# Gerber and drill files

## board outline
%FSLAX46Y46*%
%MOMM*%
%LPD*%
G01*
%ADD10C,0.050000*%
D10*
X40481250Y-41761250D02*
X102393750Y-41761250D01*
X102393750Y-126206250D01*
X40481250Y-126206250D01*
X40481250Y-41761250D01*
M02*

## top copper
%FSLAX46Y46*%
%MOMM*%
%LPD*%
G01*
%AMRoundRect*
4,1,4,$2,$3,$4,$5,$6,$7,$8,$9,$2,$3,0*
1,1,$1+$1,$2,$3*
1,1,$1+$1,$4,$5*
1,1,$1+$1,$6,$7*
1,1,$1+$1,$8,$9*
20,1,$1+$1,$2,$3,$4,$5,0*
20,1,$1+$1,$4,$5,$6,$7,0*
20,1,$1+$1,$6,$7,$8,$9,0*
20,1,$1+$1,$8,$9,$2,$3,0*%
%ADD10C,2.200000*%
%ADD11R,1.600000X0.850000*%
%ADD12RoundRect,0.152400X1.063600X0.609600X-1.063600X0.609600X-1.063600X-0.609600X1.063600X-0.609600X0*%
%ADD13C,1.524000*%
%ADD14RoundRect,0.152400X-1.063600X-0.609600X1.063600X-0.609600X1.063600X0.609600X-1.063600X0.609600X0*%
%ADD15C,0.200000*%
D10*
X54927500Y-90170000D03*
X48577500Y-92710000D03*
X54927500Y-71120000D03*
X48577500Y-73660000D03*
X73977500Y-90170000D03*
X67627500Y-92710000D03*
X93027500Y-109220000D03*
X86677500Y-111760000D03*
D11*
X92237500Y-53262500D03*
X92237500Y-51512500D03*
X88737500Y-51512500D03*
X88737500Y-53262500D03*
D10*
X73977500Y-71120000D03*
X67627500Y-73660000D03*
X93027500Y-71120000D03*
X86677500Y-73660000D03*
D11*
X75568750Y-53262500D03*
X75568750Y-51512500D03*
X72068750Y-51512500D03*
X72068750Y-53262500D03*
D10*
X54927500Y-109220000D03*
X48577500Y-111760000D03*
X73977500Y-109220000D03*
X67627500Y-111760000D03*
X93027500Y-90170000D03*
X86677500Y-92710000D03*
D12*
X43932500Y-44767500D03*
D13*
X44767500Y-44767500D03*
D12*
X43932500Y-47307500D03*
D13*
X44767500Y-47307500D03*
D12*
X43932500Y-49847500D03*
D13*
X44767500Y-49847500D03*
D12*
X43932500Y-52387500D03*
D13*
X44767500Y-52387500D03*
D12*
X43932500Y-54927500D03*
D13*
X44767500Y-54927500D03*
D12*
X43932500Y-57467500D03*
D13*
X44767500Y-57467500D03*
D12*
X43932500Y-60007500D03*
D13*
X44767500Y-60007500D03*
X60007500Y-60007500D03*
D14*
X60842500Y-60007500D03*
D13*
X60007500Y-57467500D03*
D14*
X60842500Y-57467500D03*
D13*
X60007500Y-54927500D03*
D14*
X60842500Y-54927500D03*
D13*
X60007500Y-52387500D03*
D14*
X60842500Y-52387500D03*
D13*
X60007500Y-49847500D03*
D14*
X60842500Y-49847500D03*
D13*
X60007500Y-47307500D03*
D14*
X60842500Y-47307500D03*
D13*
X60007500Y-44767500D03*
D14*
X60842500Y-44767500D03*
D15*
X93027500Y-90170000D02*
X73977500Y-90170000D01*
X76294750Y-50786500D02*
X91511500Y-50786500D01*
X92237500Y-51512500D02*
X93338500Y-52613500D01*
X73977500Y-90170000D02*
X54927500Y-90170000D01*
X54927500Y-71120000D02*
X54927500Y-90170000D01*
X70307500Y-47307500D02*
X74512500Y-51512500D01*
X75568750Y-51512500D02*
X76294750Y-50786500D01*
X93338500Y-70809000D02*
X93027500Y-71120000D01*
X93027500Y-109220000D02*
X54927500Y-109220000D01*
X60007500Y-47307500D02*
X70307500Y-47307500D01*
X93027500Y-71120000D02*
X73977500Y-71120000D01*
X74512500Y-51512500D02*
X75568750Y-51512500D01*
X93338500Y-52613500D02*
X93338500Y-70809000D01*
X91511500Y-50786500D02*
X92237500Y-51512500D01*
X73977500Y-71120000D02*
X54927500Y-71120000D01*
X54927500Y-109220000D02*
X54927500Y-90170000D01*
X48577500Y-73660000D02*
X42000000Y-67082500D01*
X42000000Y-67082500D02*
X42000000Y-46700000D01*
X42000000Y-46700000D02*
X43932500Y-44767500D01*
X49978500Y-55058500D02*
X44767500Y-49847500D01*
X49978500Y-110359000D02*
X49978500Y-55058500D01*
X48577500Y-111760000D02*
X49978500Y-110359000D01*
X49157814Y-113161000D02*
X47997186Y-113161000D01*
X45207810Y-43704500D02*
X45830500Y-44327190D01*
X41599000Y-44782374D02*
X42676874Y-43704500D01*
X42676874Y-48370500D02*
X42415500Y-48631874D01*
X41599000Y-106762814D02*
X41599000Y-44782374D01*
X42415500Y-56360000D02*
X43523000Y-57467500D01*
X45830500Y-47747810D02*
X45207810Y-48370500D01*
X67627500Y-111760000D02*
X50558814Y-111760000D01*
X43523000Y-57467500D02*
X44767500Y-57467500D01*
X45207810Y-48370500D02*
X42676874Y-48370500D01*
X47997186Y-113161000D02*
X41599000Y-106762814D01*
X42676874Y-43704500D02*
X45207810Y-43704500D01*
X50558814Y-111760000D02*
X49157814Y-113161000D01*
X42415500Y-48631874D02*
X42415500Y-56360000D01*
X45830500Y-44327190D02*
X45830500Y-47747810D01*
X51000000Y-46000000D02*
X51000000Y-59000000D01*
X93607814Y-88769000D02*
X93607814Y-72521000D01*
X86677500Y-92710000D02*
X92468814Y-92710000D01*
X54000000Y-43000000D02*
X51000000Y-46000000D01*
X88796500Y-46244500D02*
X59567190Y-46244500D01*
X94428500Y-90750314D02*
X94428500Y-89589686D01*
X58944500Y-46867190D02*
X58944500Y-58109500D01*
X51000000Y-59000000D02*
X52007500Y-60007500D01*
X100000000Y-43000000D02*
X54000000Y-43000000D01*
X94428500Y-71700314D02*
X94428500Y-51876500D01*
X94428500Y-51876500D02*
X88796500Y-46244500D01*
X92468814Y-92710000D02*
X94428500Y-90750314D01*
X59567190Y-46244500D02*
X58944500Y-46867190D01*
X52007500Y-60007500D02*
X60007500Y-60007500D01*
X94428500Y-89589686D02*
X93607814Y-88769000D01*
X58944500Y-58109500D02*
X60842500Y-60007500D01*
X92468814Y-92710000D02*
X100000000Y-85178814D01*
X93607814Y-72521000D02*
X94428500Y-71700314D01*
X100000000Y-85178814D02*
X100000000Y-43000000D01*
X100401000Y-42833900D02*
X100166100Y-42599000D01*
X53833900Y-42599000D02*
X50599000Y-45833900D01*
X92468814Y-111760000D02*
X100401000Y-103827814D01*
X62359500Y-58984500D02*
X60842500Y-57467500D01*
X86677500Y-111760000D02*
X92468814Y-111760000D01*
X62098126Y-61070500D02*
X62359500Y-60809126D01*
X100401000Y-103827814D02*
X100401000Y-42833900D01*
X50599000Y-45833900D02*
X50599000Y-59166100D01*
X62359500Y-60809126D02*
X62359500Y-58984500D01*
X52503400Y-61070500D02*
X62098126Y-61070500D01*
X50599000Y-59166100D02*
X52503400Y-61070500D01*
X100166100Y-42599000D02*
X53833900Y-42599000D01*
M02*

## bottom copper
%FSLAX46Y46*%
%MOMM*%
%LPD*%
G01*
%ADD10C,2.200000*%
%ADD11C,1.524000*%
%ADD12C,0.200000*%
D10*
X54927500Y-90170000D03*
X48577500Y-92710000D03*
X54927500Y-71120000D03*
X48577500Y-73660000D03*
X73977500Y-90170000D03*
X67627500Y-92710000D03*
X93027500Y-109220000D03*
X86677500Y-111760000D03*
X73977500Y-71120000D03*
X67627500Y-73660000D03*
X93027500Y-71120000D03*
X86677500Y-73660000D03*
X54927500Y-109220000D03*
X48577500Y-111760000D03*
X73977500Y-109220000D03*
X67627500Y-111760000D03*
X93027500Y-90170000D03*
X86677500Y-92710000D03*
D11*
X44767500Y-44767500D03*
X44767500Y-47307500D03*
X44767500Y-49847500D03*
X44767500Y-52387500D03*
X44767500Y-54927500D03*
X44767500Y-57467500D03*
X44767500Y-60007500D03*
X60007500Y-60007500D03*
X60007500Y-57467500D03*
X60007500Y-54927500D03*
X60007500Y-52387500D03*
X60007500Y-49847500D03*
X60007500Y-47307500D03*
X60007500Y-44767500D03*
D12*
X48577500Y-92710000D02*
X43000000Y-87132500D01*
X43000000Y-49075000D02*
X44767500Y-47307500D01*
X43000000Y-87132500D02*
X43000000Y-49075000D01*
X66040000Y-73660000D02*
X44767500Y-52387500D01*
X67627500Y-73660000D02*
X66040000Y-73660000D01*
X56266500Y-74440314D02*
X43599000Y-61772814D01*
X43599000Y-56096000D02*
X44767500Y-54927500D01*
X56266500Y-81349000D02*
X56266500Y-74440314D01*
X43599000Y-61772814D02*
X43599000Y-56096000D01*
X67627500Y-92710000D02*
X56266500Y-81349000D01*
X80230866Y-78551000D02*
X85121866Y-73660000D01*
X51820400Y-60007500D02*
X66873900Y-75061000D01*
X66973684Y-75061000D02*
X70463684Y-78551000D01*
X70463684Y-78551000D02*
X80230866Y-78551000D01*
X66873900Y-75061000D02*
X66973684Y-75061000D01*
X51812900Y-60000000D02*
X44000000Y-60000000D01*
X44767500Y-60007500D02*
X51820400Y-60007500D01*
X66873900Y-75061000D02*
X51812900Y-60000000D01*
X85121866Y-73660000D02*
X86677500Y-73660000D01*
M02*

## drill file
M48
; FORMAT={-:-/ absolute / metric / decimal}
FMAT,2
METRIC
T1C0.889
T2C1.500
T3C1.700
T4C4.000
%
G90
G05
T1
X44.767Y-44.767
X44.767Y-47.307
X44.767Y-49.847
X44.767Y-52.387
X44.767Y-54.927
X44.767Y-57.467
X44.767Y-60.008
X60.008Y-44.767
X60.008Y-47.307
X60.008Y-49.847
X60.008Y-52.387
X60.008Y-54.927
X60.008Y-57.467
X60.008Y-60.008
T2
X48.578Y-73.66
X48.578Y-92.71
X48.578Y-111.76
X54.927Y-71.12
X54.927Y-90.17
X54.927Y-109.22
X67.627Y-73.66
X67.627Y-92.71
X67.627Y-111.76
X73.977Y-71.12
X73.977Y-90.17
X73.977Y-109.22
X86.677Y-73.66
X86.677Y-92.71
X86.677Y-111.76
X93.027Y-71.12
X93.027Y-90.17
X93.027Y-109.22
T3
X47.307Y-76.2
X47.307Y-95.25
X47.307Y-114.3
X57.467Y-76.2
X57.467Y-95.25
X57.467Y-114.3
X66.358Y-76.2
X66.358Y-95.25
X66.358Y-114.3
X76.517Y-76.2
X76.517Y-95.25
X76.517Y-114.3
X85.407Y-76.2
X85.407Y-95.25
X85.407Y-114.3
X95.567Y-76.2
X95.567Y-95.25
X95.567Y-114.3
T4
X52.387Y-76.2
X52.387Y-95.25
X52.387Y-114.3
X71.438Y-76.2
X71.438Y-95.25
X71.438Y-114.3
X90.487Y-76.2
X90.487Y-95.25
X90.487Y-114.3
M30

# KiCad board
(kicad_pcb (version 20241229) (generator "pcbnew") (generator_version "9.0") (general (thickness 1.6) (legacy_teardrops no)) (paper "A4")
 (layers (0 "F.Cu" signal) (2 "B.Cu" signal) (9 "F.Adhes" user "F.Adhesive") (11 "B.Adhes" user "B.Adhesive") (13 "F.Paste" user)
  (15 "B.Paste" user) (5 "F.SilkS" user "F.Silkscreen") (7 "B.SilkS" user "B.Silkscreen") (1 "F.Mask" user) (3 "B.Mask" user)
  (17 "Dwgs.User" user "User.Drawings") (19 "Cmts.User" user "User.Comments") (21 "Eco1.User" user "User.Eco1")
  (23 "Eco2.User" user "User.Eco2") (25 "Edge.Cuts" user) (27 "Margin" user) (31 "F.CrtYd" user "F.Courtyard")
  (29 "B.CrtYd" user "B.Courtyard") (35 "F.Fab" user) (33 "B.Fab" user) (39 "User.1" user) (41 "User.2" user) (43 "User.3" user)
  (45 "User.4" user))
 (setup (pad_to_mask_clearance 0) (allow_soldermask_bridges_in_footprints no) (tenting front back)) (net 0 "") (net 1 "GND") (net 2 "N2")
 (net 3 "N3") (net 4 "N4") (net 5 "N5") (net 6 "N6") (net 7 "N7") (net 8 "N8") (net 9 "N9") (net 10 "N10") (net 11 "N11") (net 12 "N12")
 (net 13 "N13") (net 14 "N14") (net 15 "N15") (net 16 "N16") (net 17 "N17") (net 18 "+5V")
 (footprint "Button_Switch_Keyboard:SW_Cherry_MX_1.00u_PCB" (layer "F.Cu") (at 54.9275 90.17)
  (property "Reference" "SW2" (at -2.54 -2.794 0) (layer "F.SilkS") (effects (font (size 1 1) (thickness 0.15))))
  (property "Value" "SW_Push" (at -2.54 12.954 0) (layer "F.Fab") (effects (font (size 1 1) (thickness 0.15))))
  (pad "" np_thru_hole circle (at -7.62 5.08) (size 1.7 1.7) (drill 1.7) (layers "*.Cu" "*.Mask"))
  (pad "" np_thru_hole circle (at -2.54 5.08) (size 4 4) (drill 4) (layers "*.Cu" "*.Mask"))
  (pad "" np_thru_hole circle (at 2.54 5.08) (size 1.7 1.7) (drill 1.7) (layers "*.Cu" "*.Mask"))
  (pad "1" thru_hole circle (at 0 0) (size 2.2 2.2) (drill 1.5) (layers "*.Cu" "*.Mask") (remove_unused_layers no) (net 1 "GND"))
  (pad "2" thru_hole circle (at -6.35 2.54) (size 2.2 2.2) (drill 1.5) (layers "*.Cu" "*.Mask") (remove_unused_layers no) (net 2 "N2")))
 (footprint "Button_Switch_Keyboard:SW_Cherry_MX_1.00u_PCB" (layer "F.Cu") (at 54.9275 71.12)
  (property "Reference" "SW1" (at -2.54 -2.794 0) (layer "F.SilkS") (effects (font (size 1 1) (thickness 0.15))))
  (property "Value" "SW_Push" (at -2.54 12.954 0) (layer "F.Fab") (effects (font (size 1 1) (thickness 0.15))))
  (pad "" np_thru_hole circle (at -7.62 5.08) (size 1.7 1.7) (drill 1.7) (layers "*.Cu" "*.Mask"))
  (pad "" np_thru_hole circle (at -2.54 5.08) (size 4 4) (drill 4) (layers "*.Cu" "*.Mask"))
  (pad "" np_thru_hole circle (at 2.54 5.08) (size 1.7 1.7) (drill 1.7) (layers "*.Cu" "*.Mask"))
  (pad "1" thru_hole circle (at 0 0) (size 2.2 2.2) (drill 1.5) (layers "*.Cu" "*.Mask") (remove_unused_layers no) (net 1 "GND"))
  (pad "2" thru_hole circle (at -6.35 2.54) (size 2.2 2.2) (drill 1.5) (layers "*.Cu" "*.Mask") (remove_unused_layers no) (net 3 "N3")))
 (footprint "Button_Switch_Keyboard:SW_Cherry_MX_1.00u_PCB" (layer "F.Cu") (at 73.9775 90.17)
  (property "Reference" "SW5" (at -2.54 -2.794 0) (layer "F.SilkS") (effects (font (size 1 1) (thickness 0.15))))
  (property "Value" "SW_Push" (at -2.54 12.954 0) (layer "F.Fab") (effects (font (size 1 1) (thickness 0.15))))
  (pad "" np_thru_hole circle (at -7.62 5.08) (size 1.7 1.7) (drill 1.7) (layers "*.Cu" "*.Mask"))
  (pad "" np_thru_hole circle (at -2.54 5.08) (size 4 4) (drill 4) (layers "*.Cu" "*.Mask"))
  (pad "" np_thru_hole circle (at 2.54 5.08) (size 1.7 1.7) (drill 1.7) (layers "*.Cu" "*.Mask"))
  (pad "1" thru_hole circle (at 0 0) (size 2.2 2.2) (drill 1.5) (layers "*.Cu" "*.Mask") (remove_unused_layers no) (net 1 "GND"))
  (pad "2" thru_hole circle (at -6.35 2.54) (size 2.2 2.2) (drill 1.5) (layers "*.Cu" "*.Mask") (remove_unused_layers no) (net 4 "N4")))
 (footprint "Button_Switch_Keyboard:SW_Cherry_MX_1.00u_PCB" (layer "F.Cu") (at 93.0275 109.22)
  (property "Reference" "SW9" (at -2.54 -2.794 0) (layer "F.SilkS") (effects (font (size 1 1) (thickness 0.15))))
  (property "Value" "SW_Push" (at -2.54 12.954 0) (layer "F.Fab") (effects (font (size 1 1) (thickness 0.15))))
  (pad "" np_thru_hole circle (at -7.62 5.08) (size 1.7 1.7) (drill 1.7) (layers "*.Cu" "*.Mask"))
  (pad "" np_thru_hole circle (at -2.54 5.08) (size 4 4) (drill 4) (layers "*.Cu" "*.Mask"))
  (pad "" np_thru_hole circle (at 2.54 5.08) (size 1.7 1.7) (drill 1.7) (layers "*.Cu" "*.Mask"))
  (pad "1" thru_hole circle (at 0 0) (size 2.2 2.2) (drill 1.5) (layers "*.Cu" "*.Mask") (remove_unused_layers no) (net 1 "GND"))
  (pad "2" thru_hole circle (at -6.35 2.54) (size 2.2 2.2) (drill 1.5) (layers "*.Cu" "*.Mask") (remove_unused_layers no) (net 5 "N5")))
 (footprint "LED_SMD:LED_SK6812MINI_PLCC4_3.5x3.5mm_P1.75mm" (layer "F.Cu") (at 90.4875 52.3875 180)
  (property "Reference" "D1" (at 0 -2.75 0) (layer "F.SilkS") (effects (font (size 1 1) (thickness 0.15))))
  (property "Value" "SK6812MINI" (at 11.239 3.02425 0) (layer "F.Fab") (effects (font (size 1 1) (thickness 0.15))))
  (pad "1" smd rect (at -1.75 -0.875 180) (size 1.6 0.85) (layers "F.Cu" "F.Mask" "F.Paste") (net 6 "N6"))
  (pad "2" smd rect (at -1.75 0.875 180) (size 1.6 0.85) (layers "F.Cu" "F.Mask" "F.Paste") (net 1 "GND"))
  (pad "3" smd rect (at 1.75 0.875 180) (size 1.6 0.85) (layers "F.Cu" "F.Mask" "F.Paste") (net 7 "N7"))
  (pad "4" smd rect (at 1.75 -0.875 180) (size 1.6 0.85) (layers "F.Cu" "F.Mask" "F.Paste") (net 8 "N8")))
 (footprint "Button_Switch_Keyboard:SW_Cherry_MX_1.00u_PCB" (layer "F.Cu") (at 73.9775 71.12)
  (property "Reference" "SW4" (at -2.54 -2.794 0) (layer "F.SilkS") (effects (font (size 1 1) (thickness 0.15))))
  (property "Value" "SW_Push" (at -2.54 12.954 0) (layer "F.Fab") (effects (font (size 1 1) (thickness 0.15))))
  (pad "" np_thru_hole circle (at -7.62 5.08) (size 1.7 1.7) (drill 1.7) (layers "*.Cu" "*.Mask"))
  (pad "" np_thru_hole circle (at -2.54 5.08) (size 4 4) (drill 4) (layers "*.Cu" "*.Mask"))
  (pad "" np_thru_hole circle (at 2.54 5.08) (size 1.7 1.7) (drill 1.7) (layers "*.Cu" "*.Mask"))
  (pad "1" thru_hole circle (at 0 0) (size 2.2 2.2) (drill 1.5) (layers "*.Cu" "*.Mask") (remove_unused_layers no) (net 1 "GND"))
  (pad "2" thru_hole circle (at -6.35 2.54) (size 2.2 2.2) (drill 1.5) (layers "*.Cu" "*.Mask") (remove_unused_layers no) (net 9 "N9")))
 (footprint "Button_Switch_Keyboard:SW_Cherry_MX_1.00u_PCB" (layer "F.Cu") (at 93.0275 71.12)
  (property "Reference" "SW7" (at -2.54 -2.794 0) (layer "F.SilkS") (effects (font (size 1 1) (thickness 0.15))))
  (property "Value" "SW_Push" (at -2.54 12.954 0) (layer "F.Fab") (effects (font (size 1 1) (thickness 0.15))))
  (pad "" np_thru_hole circle (at -7.62 5.08) (size 1.7 1.7) (drill 1.7) (layers "*.Cu" "*.Mask"))
  (pad "" np_thru_hole circle (at -2.54 5.08) (size 4 4) (drill 4) (layers "*.Cu" "*.Mask"))
  (pad "" np_thru_hole circle (at 2.54 5.08) (size 1.7 1.7) (drill 1.7) (layers "*.Cu" "*.Mask"))
  (pad "1" thru_hole circle (at 0 0) (size 2.2 2.2) (drill 1.5) (layers "*.Cu" "*.Mask") (remove_unused_layers no) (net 1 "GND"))
  (pad "2" thru_hole circle (at -6.35 2.54) (size 2.2 2.2) (drill 1.5) (layers "*.Cu" "*.Mask") (remove_unused_layers no) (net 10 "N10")))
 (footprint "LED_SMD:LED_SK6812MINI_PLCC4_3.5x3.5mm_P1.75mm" (layer "F.Cu") (at 73.81875 52.3875 180)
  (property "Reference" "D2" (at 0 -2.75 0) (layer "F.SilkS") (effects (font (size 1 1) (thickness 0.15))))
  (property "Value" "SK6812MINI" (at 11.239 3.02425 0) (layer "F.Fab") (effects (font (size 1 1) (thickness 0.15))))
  (pad "1" smd rect (at -1.75 -0.875 180) (size 1.6 0.85) (layers "F.Cu" "F.Mask" "F.Paste") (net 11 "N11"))
  (pad "2" smd rect (at -1.75 0.875 180) (size 1.6 0.85) (layers "F.Cu" "F.Mask" "F.Paste") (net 1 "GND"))
  (pad "3" smd rect (at 1.75 0.875 180) (size 1.6 0.85) (layers "F.Cu" "F.Mask" "F.Paste") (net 6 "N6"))
  (pad "4" smd rect (at 1.75 -0.875 180) (size 1.6 0.85) (layers "F.Cu" "F.Mask" "F.Paste") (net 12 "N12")))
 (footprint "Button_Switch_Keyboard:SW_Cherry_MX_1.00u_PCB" (layer "F.Cu") (at 54.9275 109.22)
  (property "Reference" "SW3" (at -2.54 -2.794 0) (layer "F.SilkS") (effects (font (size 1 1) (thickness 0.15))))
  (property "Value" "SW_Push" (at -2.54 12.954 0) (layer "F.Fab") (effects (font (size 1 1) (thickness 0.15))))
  (pad "" np_thru_hole circle (at -7.62 5.08) (size 1.7 1.7) (drill 1.7) (layers "*.Cu" "*.Mask"))
  (pad "" np_thru_hole circle (at -2.54 5.08) (size 4 4) (drill 4) (layers "*.Cu" "*.Mask"))
  (pad "" np_thru_hole circle (at 2.54 5.08) (size 1.7 1.7) (drill 1.7) (layers "*.Cu" "*.Mask"))
  (pad "1" thru_hole circle (at 0 0) (size 2.2 2.2) (drill 1.5) (layers "*.Cu" "*.Mask") (remove_unused_layers no) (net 1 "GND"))
  (pad "2" thru_hole circle (at -6.35 2.54) (size 2.2 2.2) (drill 1.5) (layers "*.Cu" "*.Mask") (remove_unused_layers no) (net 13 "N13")))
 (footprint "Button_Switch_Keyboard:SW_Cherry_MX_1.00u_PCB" (layer "F.Cu") (at 73.9775 109.22)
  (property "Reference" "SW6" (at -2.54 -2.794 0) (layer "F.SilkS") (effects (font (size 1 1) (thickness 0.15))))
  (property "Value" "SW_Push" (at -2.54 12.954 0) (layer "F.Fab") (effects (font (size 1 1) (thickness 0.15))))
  (pad "" np_thru_hole circle (at -7.62 5.08) (size 1.7 1.7) (drill 1.7) (layers "*.Cu" "*.Mask"))
  (pad "" np_thru_hole circle (at -2.54 5.08) (size 4 4) (drill 4) (layers "*.Cu" "*.Mask"))
  (pad "" np_thru_hole circle (at 2.54 5.08) (size 1.7 1.7) (drill 1.7) (layers "*.Cu" "*.Mask"))
  (pad "1" thru_hole circle (at 0 0) (size 2.2 2.2) (drill 1.5) (layers "*.Cu" "*.Mask") (remove_unused_layers no) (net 1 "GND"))
  (pad "2" thru_hole circle (at -6.35 2.54) (size 2.2 2.2) (drill 1.5) (layers "*.Cu" "*.Mask") (remove_unused_layers no) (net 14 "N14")))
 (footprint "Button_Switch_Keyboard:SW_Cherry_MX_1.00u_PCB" (layer "F.Cu") (at 93.0275 90.17)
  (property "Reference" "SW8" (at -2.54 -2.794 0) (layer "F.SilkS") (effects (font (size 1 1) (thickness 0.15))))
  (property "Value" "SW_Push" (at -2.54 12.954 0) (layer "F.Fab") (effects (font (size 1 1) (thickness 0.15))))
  (pad "" np_thru_hole circle (at -7.62 5.08) (size 1.7 1.7) (drill 1.7) (layers "*.Cu" "*.Mask"))
  (pad "" np_thru_hole circle (at -2.54 5.08) (size 4 4) (drill 4) (layers "*.Cu" "*.Mask"))
  (pad "" np_thru_hole circle (at 2.54 5.08) (size 1.7 1.7) (drill 1.7) (layers "*.Cu" "*.Mask"))
  (pad "1" thru_hole circle (at 0 0) (size 2.2 2.2) (drill 1.5) (layers "*.Cu" "*.Mask") (remove_unused_layers no) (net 1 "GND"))
  (pad "2" thru_hole circle (at -6.35 2.54) (size 2.2 2.2) (drill 1.5) (layers "*.Cu" "*.Mask") (remove_unused_layers no) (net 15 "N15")))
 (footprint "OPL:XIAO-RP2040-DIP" (layer "F.Cu") (at 52.3875 52.3875)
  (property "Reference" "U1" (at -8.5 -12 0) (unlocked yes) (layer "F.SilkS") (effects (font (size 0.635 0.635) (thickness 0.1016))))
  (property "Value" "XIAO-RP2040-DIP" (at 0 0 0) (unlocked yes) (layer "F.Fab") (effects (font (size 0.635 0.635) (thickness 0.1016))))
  (pad "1" smd roundrect (at -8.455 -7.62 180) (size 2.432 1.524) (layers "F.Cu" "F.Mask") (roundrect_rratio 0.1) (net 3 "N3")
   (thermal_bridge_angle 45))
  (pad "1" thru_hole circle (at -7.62 -7.62 180) (size 1.524 1.524) (drill 0.889) (layers "*.Cu" "*.Mask") (remove_unused_layers no)
   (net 3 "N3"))
  (pad "2" smd roundrect (at -8.455 -5.08 180) (size 2.432 1.524) (layers "F.Cu" "F.Mask") (roundrect_rratio 0.1) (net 2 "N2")
   (thermal_bridge_angle 45))
  (pad "2" thru_hole circle (at -7.62 -5.08 180) (size 1.524 1.524) (drill 0.889) (layers "*.Cu" "*.Mask") (remove_unused_layers no)
   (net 2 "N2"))
  (pad "3" smd roundrect (at -8.455 -2.54 180) (size 2.432 1.524) (layers "F.Cu" "F.Mask") (roundrect_rratio 0.1) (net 13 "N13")
   (thermal_bridge_angle 45))
  (pad "3" thru_hole circle (at -7.62 -2.54 180) (size 1.524 1.524) (drill 0.889) (layers "*.Cu" "*.Mask") (remove_unused_layers no)
   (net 13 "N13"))
  (pad "4" smd roundrect (at -8.455 0 180) (size 2.432 1.524) (layers "F.Cu" "F.Mask") (roundrect_rratio 0.1) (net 9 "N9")
   (thermal_bridge_angle 45))
  (pad "4" thru_hole circle (at -7.62 0 180) (size 1.524 1.524) (drill 0.889) (layers "*.Cu" "*.Mask") (remove_unused_layers no)
   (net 9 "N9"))
  (pad "5" smd roundrect (at -8.455 2.54 180) (size 2.432 1.524) (layers "F.Cu" "F.Mask") (roundrect_rratio 0.1) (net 4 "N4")
   (thermal_bridge_angle 45))
  (pad "5" thru_hole circle (at -7.62 2.54 180) (size 1.524 1.524) (drill 0.889) (layers "*.Cu" "*.Mask") (remove_unused_layers no)
   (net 4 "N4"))
  (pad "6" smd roundrect (at -8.455 5.08 180) (size 2.432 1.524) (layers "F.Cu" "F.Mask") (roundrect_rratio 0.1) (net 14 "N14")
   (thermal_bridge_angle 45))
  (pad "6" thru_hole circle (at -7.62 5.08 180) (size 1.524 1.524) (drill 0.889) (layers "*.Cu" "*.Mask") (remove_unused_layers no)
   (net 14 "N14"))
  (pad "7" smd roundrect (at -8.455 7.62 180) (size 2.432 1.524) (layers "F.Cu" "F.Mask") (roundrect_rratio 0.1) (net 10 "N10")
   (thermal_bridge_angle 45))
  (pad "7" thru_hole circle (at -7.62 7.62 180) (size 1.524 1.524) (drill 0.889) (layers "*.Cu" "*.Mask") (remove_unused_layers no)
   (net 10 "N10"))
  (pad "8" thru_hole circle (at 7.62 7.62) (size 1.524 1.524) (drill 0.889) (layers "*.Cu" "*.Mask") (remove_unused_layers no)
   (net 15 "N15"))
  (pad "8" smd roundrect (at 8.455 7.62) (size 2.432 1.524) (layers "F.Cu" "F.Mask") (roundrect_rratio 0.1) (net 15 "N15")
   (thermal_bridge_angle 45))
  (pad "9" thru_hole circle (at 7.62 5.08) (size 1.524 1.524) (drill 0.889) (layers "*.Cu" "*.Mask") (remove_unused_layers no) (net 5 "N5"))
  (pad "9" smd roundrect (at 8.455 5.08) (size 2.432 1.524) (layers "F.Cu" "F.Mask") (roundrect_rratio 0.1) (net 5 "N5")
   (thermal_bridge_angle 45))
  (pad "10" thru_hole circle (at 7.62 2.54) (size 1.524 1.524) (drill 0.889) (layers "*.Cu" "*.Mask") (remove_unused_layers no)
   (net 11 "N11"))
  (pad "10" smd roundrect (at 8.455 2.54) (size 2.432 1.524) (layers "F.Cu" "F.Mask") (roundrect_rratio 0.1) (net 11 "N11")
   (thermal_bridge_angle 45))
  (pad "11" thru_hole circle (at 7.62 0) (size 1.524 1.524) (drill 0.889) (layers "*.Cu" "*.Mask") (remove_unused_layers no) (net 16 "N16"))
  (pad "11" smd roundrect (at 8.455 0) (size 2.432 1.524) (layers "F.Cu" "F.Mask") (roundrect_rratio 0.1) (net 16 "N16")
   (thermal_bridge_angle 45))
  (pad "12" thru_hole circle (at 7.62 -2.54) (size 1.524 1.524) (drill 0.889) (layers "*.Cu" "*.Mask") (remove_unused_layers no)
   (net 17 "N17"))
  (pad "12" smd roundrect (at 8.455 -2.54) (size 2.432 1.524) (layers "F.Cu" "F.Mask") (roundrect_rratio 0.1) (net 17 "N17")
   (thermal_bridge_angle 45))
  (pad "13" thru_hole circle (at 7.62 -5.08) (size 1.524 1.524) (drill 0.889) (layers "*.Cu" "*.Mask") (remove_unused_layers no)
   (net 1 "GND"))
  (pad "13" smd roundrect (at 8.455 -5.08) (size 2.432 1.524) (layers "F.Cu" "F.Mask") (roundrect_rratio 0.1) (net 1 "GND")
   (thermal_bridge_angle 45))
  (pad "14" thru_hole circle (at 7.62 -7.62) (size 1.524 1.524) (drill 0.889) (layers "*.Cu" "*.Mask") (remove_unused_layers no)
   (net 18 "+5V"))
  (pad "14" smd roundrect (at 8.455 -7.62) (size 2.432 1.524) (layers "F.Cu" "F.Mask") (roundrect_rratio 0.1) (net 18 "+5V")
   (thermal_bridge_angle 45)))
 (gr_rect (start 40.48125 41.76125) (end 102.39375 126.20625) (stroke (width 0.05) (type default)) (fill no) (layer "Edge.Cuts"))
 (segment (start 93.0275 90.17) (end 73.9775 90.17) (width 0.2) (layer "F.Cu") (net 1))
 (segment (start 76.29475 50.7865) (end 91.5115 50.7865) (width 0.2) (layer "F.Cu") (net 1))
 (segment (start 92.2375 51.5125) (end 93.3385 52.6135) (width 0.2) (layer "F.Cu") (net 1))
 (segment (start 73.9775 90.17) (end 54.9275 90.17) (width 0.2) (layer "F.Cu") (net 1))
 (segment (start 54.9275 71.12) (end 54.9275 90.17) (width 0.2) (layer "F.Cu") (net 1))
 (segment (start 70.3075 47.3075) (end 74.5125 51.5125) (width 0.2) (layer "F.Cu") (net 1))
 (segment (start 75.56875 51.5125) (end 76.29475 50.7865) (width 0.2) (layer "F.Cu") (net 1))
 (segment (start 93.3385 70.809) (end 93.0275 71.12) (width 0.2) (layer "F.Cu") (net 1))
 (segment (start 93.0275 109.22) (end 54.9275 109.22) (width 0.2) (layer "F.Cu") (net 1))
 (segment (start 60.0075 47.3075) (end 70.3075 47.3075) (width 0.2) (layer "F.Cu") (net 1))
 (segment (start 93.0275 71.12) (end 73.9775 71.12) (width 0.2) (layer "F.Cu") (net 1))
 (segment (start 74.5125 51.5125) (end 75.56875 51.5125) (width 0.2) (layer "F.Cu") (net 1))
 (segment (start 93.3385 52.6135) (end 93.3385 70.809) (width 0.2) (layer "F.Cu") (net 1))
 (segment (start 91.5115 50.7865) (end 92.2375 51.5125) (width 0.2) (layer "F.Cu") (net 1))
 (segment (start 73.9775 71.12) (end 54.9275 71.12) (width 0.2) (layer "F.Cu") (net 1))
 (segment (start 54.9275 109.22) (end 54.9275 90.17) (width 0.2) (layer "F.Cu") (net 1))
 (segment (start 48.5775 73.66) (end 42 67.0825) (width 0.2) (layer "F.Cu") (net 3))
 (segment (start 42 67.0825) (end 42 46.7) (width 0.2) (layer "F.Cu") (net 3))
 (segment (start 42 46.7) (end 43.9325 44.7675) (width 0.2) (layer "F.Cu") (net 3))
 (segment (start 48.5775 92.71) (end 43 87.1325) (width 0.2) (layer "B.Cu") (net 2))
 (segment (start 43 49.075) (end 44.7675 47.3075) (width 0.2) (layer "B.Cu") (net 2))
 (segment (start 43 87.1325) (end 43 49.075) (width 0.2) (layer "B.Cu") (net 2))
 (segment (start 49.9785 55.0585) (end 44.7675 49.8475) (width 0.2) (layer "F.Cu") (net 13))
 (segment (start 49.9785 110.359) (end 49.9785 55.0585) (width 0.2) (layer "F.Cu") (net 13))
 (segment (start 48.5775 111.76) (end 49.9785 110.359) (width 0.2) (layer "F.Cu") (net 13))
 (segment (start 66.04 73.66) (end 44.7675 52.3875) (width 0.2) (layer "B.Cu") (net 9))
 (segment (start 67.6275 73.66) (end 66.04 73.66) (width 0.2) (layer "B.Cu") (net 9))
 (segment (start 56.2665 74.440314) (end 43.599 61.772814) (width 0.2) (layer "B.Cu") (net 4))
 (segment (start 43.599 56.096) (end 44.7675 54.9275) (width 0.2) (layer "B.Cu") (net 4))
 (segment (start 56.2665 81.349) (end 56.2665 74.440314) (width 0.2) (layer "B.Cu") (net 4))
 (segment (start 43.599 61.772814) (end 43.599 56.096) (width 0.2) (layer "B.Cu") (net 4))
 (segment (start 67.6275 92.71) (end 56.2665 81.349) (width 0.2) (layer "B.Cu") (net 4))
 (segment (start 49.157814 113.161) (end 47.997186 113.161) (width 0.2) (layer "F.Cu") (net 14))
 (segment (start 45.20781 43.7045) (end 45.8305 44.32719) (width 0.2) (layer "F.Cu") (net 14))
 (segment (start 41.599 44.782374) (end 42.676874 43.7045) (width 0.2) (layer "F.Cu") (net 14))
 (segment (start 42.676874 48.3705) (end 42.4155 48.631874) (width 0.2) (layer "F.Cu") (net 14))
 (segment (start 41.599 106.762814) (end 41.599 44.782374) (width 0.2) (layer "F.Cu") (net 14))
 (segment (start 42.4155 56.36) (end 43.523 57.4675) (width 0.2) (layer "F.Cu") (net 14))
 (segment (start 45.8305 47.74781) (end 45.20781 48.3705) (width 0.2) (layer "F.Cu") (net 14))
 (segment (start 67.6275 111.76) (end 50.558814 111.76) (width 0.2) (layer "F.Cu") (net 14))
 (segment (start 43.523 57.4675) (end 44.7675 57.4675) (width 0.2) (layer "F.Cu") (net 14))
 (segment (start 45.20781 48.3705) (end 42.676874 48.3705) (width 0.2) (layer "F.Cu") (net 14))
 (segment (start 47.997186 113.161) (end 41.599 106.762814) (width 0.2) (layer "F.Cu") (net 14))
 (segment (start 42.676874 43.7045) (end 45.20781 43.7045) (width 0.2) (layer "F.Cu") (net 14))
 (segment (start 50.558814 111.76) (end 49.157814 113.161) (width 0.2) (layer "F.Cu") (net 14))
 (segment (start 42.4155 48.631874) (end 42.4155 56.36) (width 0.2) (layer "F.Cu") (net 14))
 (segment (start 45.8305 44.32719) (end 45.8305 47.74781) (width 0.2) (layer "F.Cu") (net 14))
 (segment (start 80.230866 78.551) (end 85.121866 73.66) (width 0.2) (layer "B.Cu") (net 10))
 (segment (start 51.8204 60.0075) (end 66.8739 75.061) (width 0.2) (layer "B.Cu") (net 10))
 (segment (start 66.973684 75.061) (end 70.463684 78.551) (width 0.2) (layer "B.Cu") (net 10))
 (segment (start 70.463684 78.551) (end 80.230866 78.551) (width 0.2) (layer "B.Cu") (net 10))
 (segment (start 66.8739 75.061) (end 66.973684 75.061) (width 0.2) (layer "B.Cu") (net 10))
 (segment (start 51.8129 60) (end 44 60) (width 0.2) (layer "B.Cu") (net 10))
 (segment (start 44.7675 60.0075) (end 51.8204 60.0075) (width 0.2) (layer "B.Cu") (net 10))
 (segment (start 66.8739 75.061) (end 51.8129 60) (width 0.2) (layer "B.Cu") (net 10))
 (segment (start 85.121866 73.66) (end 86.6775 73.66) (width 0.2) (layer "B.Cu") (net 10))
 (segment (start 51 46) (end 51 59) (width 0.2) (layer "F.Cu") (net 15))
 (segment (start 93.607814 88.769) (end 93.607814 72.521) (width 0.2) (layer "F.Cu") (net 15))
 (segment (start 86.6775 92.71) (end 92.468814 92.71) (width 0.2) (layer "F.Cu") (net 15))
 (segment (start 54 43) (end 51 46) (width 0.2) (layer "F.Cu") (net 15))
 (segment (start 88.7965 46.2445) (end 59.56719 46.2445) (width 0.2) (layer "F.Cu") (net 15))
 (segment (start 94.4285 90.750314) (end 94.4285 89.589686) (width 0.2) (layer "F.Cu") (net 15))
 (segment (start 58.9445 46.86719) (end 58.9445 58.1095) (width 0.2) (layer "F.Cu") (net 15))
 (segment (start 51 59) (end 52.0075 60.0075) (width 0.2) (layer "F.Cu") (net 15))
 (segment (start 100 43) (end 54 43) (width 0.2) (layer "F.Cu") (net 15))
 (segment (start 94.4285 71.700314) (end 94.4285 51.8765) (width 0.2) (layer "F.Cu") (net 15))
 (segment (start 94.4285 51.8765) (end 88.7965 46.2445) (width 0.2) (layer "F.Cu") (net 15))
 (segment (start 92.468814 92.71) (end 94.4285 90.750314) (width 0.2) (layer "F.Cu") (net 15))
 (segment (start 59.56719 46.2445) (end 58.9445 46.86719) (width 0.2) (layer "F.Cu") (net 15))
 (segment (start 52.0075 60.0075) (end 60.0075 60.0075) (width 0.2) (layer "F.Cu") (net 15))
 (segment (start 94.4285 89.589686) (end 93.607814 88.769) (width 0.2) (layer "F.Cu") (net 15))
 (segment (start 58.9445 58.1095) (end 60.8425 60.0075) (width 0.2) (layer "F.Cu") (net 15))
 (segment (start 92.468814 92.71) (end 100 85.178814) (width 0.2) (layer "F.Cu") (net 15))
 (segment (start 93.607814 72.521) (end 94.4285 71.700314) (width 0.2) (layer "F.Cu") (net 15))
 (segment (start 100 85.178814) (end 100 43) (width 0.2) (layer "F.Cu") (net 15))
 (segment (start 100.401 42.8339) (end 100.1661 42.599) (width 0.2) (layer "F.Cu") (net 5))
 (segment (start 53.8339 42.599) (end 50.599 45.8339) (width 0.2) (layer "F.Cu") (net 5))
 (segment (start 92.468814 111.76) (end 100.401 103.827814) (width 0.2) (layer "F.Cu") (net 5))
 (segment (start 62.3595 58.9845) (end 60.8425 57.4675) (width 0.2) (layer "F.Cu") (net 5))
 (segment (start 86.6775 111.76) (end 92.468814 111.76) (width 0.2) (layer "F.Cu") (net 5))
 (segment (start 62.098126 61.0705) (end 62.3595 60.809126) (width 0.2) (layer "F.Cu") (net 5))
 (segment (start 100.401 103.827814) (end 100.401 42.8339) (width 0.2) (layer "F.Cu") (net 5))
 (segment (start 50.599 45.8339) (end 50.599 59.1661) (width 0.2) (layer "F.Cu") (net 5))
 (segment (start 62.3595 60.809126) (end 62.3595 58.9845) (width 0.2) (layer "F.Cu") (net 5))
 (segment (start 52.5034 61.0705) (end 62.098126 61.0705) (width 0.2) (layer "F.Cu") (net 5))
 (segment (start 50.599 59.1661) (end 52.5034 61.0705) (width 0.2) (layer "F.Cu") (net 5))
 (segment (start 100.1661 42.599) (end 53.8339 42.599) (width 0.2) (layer "F.Cu") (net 5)))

